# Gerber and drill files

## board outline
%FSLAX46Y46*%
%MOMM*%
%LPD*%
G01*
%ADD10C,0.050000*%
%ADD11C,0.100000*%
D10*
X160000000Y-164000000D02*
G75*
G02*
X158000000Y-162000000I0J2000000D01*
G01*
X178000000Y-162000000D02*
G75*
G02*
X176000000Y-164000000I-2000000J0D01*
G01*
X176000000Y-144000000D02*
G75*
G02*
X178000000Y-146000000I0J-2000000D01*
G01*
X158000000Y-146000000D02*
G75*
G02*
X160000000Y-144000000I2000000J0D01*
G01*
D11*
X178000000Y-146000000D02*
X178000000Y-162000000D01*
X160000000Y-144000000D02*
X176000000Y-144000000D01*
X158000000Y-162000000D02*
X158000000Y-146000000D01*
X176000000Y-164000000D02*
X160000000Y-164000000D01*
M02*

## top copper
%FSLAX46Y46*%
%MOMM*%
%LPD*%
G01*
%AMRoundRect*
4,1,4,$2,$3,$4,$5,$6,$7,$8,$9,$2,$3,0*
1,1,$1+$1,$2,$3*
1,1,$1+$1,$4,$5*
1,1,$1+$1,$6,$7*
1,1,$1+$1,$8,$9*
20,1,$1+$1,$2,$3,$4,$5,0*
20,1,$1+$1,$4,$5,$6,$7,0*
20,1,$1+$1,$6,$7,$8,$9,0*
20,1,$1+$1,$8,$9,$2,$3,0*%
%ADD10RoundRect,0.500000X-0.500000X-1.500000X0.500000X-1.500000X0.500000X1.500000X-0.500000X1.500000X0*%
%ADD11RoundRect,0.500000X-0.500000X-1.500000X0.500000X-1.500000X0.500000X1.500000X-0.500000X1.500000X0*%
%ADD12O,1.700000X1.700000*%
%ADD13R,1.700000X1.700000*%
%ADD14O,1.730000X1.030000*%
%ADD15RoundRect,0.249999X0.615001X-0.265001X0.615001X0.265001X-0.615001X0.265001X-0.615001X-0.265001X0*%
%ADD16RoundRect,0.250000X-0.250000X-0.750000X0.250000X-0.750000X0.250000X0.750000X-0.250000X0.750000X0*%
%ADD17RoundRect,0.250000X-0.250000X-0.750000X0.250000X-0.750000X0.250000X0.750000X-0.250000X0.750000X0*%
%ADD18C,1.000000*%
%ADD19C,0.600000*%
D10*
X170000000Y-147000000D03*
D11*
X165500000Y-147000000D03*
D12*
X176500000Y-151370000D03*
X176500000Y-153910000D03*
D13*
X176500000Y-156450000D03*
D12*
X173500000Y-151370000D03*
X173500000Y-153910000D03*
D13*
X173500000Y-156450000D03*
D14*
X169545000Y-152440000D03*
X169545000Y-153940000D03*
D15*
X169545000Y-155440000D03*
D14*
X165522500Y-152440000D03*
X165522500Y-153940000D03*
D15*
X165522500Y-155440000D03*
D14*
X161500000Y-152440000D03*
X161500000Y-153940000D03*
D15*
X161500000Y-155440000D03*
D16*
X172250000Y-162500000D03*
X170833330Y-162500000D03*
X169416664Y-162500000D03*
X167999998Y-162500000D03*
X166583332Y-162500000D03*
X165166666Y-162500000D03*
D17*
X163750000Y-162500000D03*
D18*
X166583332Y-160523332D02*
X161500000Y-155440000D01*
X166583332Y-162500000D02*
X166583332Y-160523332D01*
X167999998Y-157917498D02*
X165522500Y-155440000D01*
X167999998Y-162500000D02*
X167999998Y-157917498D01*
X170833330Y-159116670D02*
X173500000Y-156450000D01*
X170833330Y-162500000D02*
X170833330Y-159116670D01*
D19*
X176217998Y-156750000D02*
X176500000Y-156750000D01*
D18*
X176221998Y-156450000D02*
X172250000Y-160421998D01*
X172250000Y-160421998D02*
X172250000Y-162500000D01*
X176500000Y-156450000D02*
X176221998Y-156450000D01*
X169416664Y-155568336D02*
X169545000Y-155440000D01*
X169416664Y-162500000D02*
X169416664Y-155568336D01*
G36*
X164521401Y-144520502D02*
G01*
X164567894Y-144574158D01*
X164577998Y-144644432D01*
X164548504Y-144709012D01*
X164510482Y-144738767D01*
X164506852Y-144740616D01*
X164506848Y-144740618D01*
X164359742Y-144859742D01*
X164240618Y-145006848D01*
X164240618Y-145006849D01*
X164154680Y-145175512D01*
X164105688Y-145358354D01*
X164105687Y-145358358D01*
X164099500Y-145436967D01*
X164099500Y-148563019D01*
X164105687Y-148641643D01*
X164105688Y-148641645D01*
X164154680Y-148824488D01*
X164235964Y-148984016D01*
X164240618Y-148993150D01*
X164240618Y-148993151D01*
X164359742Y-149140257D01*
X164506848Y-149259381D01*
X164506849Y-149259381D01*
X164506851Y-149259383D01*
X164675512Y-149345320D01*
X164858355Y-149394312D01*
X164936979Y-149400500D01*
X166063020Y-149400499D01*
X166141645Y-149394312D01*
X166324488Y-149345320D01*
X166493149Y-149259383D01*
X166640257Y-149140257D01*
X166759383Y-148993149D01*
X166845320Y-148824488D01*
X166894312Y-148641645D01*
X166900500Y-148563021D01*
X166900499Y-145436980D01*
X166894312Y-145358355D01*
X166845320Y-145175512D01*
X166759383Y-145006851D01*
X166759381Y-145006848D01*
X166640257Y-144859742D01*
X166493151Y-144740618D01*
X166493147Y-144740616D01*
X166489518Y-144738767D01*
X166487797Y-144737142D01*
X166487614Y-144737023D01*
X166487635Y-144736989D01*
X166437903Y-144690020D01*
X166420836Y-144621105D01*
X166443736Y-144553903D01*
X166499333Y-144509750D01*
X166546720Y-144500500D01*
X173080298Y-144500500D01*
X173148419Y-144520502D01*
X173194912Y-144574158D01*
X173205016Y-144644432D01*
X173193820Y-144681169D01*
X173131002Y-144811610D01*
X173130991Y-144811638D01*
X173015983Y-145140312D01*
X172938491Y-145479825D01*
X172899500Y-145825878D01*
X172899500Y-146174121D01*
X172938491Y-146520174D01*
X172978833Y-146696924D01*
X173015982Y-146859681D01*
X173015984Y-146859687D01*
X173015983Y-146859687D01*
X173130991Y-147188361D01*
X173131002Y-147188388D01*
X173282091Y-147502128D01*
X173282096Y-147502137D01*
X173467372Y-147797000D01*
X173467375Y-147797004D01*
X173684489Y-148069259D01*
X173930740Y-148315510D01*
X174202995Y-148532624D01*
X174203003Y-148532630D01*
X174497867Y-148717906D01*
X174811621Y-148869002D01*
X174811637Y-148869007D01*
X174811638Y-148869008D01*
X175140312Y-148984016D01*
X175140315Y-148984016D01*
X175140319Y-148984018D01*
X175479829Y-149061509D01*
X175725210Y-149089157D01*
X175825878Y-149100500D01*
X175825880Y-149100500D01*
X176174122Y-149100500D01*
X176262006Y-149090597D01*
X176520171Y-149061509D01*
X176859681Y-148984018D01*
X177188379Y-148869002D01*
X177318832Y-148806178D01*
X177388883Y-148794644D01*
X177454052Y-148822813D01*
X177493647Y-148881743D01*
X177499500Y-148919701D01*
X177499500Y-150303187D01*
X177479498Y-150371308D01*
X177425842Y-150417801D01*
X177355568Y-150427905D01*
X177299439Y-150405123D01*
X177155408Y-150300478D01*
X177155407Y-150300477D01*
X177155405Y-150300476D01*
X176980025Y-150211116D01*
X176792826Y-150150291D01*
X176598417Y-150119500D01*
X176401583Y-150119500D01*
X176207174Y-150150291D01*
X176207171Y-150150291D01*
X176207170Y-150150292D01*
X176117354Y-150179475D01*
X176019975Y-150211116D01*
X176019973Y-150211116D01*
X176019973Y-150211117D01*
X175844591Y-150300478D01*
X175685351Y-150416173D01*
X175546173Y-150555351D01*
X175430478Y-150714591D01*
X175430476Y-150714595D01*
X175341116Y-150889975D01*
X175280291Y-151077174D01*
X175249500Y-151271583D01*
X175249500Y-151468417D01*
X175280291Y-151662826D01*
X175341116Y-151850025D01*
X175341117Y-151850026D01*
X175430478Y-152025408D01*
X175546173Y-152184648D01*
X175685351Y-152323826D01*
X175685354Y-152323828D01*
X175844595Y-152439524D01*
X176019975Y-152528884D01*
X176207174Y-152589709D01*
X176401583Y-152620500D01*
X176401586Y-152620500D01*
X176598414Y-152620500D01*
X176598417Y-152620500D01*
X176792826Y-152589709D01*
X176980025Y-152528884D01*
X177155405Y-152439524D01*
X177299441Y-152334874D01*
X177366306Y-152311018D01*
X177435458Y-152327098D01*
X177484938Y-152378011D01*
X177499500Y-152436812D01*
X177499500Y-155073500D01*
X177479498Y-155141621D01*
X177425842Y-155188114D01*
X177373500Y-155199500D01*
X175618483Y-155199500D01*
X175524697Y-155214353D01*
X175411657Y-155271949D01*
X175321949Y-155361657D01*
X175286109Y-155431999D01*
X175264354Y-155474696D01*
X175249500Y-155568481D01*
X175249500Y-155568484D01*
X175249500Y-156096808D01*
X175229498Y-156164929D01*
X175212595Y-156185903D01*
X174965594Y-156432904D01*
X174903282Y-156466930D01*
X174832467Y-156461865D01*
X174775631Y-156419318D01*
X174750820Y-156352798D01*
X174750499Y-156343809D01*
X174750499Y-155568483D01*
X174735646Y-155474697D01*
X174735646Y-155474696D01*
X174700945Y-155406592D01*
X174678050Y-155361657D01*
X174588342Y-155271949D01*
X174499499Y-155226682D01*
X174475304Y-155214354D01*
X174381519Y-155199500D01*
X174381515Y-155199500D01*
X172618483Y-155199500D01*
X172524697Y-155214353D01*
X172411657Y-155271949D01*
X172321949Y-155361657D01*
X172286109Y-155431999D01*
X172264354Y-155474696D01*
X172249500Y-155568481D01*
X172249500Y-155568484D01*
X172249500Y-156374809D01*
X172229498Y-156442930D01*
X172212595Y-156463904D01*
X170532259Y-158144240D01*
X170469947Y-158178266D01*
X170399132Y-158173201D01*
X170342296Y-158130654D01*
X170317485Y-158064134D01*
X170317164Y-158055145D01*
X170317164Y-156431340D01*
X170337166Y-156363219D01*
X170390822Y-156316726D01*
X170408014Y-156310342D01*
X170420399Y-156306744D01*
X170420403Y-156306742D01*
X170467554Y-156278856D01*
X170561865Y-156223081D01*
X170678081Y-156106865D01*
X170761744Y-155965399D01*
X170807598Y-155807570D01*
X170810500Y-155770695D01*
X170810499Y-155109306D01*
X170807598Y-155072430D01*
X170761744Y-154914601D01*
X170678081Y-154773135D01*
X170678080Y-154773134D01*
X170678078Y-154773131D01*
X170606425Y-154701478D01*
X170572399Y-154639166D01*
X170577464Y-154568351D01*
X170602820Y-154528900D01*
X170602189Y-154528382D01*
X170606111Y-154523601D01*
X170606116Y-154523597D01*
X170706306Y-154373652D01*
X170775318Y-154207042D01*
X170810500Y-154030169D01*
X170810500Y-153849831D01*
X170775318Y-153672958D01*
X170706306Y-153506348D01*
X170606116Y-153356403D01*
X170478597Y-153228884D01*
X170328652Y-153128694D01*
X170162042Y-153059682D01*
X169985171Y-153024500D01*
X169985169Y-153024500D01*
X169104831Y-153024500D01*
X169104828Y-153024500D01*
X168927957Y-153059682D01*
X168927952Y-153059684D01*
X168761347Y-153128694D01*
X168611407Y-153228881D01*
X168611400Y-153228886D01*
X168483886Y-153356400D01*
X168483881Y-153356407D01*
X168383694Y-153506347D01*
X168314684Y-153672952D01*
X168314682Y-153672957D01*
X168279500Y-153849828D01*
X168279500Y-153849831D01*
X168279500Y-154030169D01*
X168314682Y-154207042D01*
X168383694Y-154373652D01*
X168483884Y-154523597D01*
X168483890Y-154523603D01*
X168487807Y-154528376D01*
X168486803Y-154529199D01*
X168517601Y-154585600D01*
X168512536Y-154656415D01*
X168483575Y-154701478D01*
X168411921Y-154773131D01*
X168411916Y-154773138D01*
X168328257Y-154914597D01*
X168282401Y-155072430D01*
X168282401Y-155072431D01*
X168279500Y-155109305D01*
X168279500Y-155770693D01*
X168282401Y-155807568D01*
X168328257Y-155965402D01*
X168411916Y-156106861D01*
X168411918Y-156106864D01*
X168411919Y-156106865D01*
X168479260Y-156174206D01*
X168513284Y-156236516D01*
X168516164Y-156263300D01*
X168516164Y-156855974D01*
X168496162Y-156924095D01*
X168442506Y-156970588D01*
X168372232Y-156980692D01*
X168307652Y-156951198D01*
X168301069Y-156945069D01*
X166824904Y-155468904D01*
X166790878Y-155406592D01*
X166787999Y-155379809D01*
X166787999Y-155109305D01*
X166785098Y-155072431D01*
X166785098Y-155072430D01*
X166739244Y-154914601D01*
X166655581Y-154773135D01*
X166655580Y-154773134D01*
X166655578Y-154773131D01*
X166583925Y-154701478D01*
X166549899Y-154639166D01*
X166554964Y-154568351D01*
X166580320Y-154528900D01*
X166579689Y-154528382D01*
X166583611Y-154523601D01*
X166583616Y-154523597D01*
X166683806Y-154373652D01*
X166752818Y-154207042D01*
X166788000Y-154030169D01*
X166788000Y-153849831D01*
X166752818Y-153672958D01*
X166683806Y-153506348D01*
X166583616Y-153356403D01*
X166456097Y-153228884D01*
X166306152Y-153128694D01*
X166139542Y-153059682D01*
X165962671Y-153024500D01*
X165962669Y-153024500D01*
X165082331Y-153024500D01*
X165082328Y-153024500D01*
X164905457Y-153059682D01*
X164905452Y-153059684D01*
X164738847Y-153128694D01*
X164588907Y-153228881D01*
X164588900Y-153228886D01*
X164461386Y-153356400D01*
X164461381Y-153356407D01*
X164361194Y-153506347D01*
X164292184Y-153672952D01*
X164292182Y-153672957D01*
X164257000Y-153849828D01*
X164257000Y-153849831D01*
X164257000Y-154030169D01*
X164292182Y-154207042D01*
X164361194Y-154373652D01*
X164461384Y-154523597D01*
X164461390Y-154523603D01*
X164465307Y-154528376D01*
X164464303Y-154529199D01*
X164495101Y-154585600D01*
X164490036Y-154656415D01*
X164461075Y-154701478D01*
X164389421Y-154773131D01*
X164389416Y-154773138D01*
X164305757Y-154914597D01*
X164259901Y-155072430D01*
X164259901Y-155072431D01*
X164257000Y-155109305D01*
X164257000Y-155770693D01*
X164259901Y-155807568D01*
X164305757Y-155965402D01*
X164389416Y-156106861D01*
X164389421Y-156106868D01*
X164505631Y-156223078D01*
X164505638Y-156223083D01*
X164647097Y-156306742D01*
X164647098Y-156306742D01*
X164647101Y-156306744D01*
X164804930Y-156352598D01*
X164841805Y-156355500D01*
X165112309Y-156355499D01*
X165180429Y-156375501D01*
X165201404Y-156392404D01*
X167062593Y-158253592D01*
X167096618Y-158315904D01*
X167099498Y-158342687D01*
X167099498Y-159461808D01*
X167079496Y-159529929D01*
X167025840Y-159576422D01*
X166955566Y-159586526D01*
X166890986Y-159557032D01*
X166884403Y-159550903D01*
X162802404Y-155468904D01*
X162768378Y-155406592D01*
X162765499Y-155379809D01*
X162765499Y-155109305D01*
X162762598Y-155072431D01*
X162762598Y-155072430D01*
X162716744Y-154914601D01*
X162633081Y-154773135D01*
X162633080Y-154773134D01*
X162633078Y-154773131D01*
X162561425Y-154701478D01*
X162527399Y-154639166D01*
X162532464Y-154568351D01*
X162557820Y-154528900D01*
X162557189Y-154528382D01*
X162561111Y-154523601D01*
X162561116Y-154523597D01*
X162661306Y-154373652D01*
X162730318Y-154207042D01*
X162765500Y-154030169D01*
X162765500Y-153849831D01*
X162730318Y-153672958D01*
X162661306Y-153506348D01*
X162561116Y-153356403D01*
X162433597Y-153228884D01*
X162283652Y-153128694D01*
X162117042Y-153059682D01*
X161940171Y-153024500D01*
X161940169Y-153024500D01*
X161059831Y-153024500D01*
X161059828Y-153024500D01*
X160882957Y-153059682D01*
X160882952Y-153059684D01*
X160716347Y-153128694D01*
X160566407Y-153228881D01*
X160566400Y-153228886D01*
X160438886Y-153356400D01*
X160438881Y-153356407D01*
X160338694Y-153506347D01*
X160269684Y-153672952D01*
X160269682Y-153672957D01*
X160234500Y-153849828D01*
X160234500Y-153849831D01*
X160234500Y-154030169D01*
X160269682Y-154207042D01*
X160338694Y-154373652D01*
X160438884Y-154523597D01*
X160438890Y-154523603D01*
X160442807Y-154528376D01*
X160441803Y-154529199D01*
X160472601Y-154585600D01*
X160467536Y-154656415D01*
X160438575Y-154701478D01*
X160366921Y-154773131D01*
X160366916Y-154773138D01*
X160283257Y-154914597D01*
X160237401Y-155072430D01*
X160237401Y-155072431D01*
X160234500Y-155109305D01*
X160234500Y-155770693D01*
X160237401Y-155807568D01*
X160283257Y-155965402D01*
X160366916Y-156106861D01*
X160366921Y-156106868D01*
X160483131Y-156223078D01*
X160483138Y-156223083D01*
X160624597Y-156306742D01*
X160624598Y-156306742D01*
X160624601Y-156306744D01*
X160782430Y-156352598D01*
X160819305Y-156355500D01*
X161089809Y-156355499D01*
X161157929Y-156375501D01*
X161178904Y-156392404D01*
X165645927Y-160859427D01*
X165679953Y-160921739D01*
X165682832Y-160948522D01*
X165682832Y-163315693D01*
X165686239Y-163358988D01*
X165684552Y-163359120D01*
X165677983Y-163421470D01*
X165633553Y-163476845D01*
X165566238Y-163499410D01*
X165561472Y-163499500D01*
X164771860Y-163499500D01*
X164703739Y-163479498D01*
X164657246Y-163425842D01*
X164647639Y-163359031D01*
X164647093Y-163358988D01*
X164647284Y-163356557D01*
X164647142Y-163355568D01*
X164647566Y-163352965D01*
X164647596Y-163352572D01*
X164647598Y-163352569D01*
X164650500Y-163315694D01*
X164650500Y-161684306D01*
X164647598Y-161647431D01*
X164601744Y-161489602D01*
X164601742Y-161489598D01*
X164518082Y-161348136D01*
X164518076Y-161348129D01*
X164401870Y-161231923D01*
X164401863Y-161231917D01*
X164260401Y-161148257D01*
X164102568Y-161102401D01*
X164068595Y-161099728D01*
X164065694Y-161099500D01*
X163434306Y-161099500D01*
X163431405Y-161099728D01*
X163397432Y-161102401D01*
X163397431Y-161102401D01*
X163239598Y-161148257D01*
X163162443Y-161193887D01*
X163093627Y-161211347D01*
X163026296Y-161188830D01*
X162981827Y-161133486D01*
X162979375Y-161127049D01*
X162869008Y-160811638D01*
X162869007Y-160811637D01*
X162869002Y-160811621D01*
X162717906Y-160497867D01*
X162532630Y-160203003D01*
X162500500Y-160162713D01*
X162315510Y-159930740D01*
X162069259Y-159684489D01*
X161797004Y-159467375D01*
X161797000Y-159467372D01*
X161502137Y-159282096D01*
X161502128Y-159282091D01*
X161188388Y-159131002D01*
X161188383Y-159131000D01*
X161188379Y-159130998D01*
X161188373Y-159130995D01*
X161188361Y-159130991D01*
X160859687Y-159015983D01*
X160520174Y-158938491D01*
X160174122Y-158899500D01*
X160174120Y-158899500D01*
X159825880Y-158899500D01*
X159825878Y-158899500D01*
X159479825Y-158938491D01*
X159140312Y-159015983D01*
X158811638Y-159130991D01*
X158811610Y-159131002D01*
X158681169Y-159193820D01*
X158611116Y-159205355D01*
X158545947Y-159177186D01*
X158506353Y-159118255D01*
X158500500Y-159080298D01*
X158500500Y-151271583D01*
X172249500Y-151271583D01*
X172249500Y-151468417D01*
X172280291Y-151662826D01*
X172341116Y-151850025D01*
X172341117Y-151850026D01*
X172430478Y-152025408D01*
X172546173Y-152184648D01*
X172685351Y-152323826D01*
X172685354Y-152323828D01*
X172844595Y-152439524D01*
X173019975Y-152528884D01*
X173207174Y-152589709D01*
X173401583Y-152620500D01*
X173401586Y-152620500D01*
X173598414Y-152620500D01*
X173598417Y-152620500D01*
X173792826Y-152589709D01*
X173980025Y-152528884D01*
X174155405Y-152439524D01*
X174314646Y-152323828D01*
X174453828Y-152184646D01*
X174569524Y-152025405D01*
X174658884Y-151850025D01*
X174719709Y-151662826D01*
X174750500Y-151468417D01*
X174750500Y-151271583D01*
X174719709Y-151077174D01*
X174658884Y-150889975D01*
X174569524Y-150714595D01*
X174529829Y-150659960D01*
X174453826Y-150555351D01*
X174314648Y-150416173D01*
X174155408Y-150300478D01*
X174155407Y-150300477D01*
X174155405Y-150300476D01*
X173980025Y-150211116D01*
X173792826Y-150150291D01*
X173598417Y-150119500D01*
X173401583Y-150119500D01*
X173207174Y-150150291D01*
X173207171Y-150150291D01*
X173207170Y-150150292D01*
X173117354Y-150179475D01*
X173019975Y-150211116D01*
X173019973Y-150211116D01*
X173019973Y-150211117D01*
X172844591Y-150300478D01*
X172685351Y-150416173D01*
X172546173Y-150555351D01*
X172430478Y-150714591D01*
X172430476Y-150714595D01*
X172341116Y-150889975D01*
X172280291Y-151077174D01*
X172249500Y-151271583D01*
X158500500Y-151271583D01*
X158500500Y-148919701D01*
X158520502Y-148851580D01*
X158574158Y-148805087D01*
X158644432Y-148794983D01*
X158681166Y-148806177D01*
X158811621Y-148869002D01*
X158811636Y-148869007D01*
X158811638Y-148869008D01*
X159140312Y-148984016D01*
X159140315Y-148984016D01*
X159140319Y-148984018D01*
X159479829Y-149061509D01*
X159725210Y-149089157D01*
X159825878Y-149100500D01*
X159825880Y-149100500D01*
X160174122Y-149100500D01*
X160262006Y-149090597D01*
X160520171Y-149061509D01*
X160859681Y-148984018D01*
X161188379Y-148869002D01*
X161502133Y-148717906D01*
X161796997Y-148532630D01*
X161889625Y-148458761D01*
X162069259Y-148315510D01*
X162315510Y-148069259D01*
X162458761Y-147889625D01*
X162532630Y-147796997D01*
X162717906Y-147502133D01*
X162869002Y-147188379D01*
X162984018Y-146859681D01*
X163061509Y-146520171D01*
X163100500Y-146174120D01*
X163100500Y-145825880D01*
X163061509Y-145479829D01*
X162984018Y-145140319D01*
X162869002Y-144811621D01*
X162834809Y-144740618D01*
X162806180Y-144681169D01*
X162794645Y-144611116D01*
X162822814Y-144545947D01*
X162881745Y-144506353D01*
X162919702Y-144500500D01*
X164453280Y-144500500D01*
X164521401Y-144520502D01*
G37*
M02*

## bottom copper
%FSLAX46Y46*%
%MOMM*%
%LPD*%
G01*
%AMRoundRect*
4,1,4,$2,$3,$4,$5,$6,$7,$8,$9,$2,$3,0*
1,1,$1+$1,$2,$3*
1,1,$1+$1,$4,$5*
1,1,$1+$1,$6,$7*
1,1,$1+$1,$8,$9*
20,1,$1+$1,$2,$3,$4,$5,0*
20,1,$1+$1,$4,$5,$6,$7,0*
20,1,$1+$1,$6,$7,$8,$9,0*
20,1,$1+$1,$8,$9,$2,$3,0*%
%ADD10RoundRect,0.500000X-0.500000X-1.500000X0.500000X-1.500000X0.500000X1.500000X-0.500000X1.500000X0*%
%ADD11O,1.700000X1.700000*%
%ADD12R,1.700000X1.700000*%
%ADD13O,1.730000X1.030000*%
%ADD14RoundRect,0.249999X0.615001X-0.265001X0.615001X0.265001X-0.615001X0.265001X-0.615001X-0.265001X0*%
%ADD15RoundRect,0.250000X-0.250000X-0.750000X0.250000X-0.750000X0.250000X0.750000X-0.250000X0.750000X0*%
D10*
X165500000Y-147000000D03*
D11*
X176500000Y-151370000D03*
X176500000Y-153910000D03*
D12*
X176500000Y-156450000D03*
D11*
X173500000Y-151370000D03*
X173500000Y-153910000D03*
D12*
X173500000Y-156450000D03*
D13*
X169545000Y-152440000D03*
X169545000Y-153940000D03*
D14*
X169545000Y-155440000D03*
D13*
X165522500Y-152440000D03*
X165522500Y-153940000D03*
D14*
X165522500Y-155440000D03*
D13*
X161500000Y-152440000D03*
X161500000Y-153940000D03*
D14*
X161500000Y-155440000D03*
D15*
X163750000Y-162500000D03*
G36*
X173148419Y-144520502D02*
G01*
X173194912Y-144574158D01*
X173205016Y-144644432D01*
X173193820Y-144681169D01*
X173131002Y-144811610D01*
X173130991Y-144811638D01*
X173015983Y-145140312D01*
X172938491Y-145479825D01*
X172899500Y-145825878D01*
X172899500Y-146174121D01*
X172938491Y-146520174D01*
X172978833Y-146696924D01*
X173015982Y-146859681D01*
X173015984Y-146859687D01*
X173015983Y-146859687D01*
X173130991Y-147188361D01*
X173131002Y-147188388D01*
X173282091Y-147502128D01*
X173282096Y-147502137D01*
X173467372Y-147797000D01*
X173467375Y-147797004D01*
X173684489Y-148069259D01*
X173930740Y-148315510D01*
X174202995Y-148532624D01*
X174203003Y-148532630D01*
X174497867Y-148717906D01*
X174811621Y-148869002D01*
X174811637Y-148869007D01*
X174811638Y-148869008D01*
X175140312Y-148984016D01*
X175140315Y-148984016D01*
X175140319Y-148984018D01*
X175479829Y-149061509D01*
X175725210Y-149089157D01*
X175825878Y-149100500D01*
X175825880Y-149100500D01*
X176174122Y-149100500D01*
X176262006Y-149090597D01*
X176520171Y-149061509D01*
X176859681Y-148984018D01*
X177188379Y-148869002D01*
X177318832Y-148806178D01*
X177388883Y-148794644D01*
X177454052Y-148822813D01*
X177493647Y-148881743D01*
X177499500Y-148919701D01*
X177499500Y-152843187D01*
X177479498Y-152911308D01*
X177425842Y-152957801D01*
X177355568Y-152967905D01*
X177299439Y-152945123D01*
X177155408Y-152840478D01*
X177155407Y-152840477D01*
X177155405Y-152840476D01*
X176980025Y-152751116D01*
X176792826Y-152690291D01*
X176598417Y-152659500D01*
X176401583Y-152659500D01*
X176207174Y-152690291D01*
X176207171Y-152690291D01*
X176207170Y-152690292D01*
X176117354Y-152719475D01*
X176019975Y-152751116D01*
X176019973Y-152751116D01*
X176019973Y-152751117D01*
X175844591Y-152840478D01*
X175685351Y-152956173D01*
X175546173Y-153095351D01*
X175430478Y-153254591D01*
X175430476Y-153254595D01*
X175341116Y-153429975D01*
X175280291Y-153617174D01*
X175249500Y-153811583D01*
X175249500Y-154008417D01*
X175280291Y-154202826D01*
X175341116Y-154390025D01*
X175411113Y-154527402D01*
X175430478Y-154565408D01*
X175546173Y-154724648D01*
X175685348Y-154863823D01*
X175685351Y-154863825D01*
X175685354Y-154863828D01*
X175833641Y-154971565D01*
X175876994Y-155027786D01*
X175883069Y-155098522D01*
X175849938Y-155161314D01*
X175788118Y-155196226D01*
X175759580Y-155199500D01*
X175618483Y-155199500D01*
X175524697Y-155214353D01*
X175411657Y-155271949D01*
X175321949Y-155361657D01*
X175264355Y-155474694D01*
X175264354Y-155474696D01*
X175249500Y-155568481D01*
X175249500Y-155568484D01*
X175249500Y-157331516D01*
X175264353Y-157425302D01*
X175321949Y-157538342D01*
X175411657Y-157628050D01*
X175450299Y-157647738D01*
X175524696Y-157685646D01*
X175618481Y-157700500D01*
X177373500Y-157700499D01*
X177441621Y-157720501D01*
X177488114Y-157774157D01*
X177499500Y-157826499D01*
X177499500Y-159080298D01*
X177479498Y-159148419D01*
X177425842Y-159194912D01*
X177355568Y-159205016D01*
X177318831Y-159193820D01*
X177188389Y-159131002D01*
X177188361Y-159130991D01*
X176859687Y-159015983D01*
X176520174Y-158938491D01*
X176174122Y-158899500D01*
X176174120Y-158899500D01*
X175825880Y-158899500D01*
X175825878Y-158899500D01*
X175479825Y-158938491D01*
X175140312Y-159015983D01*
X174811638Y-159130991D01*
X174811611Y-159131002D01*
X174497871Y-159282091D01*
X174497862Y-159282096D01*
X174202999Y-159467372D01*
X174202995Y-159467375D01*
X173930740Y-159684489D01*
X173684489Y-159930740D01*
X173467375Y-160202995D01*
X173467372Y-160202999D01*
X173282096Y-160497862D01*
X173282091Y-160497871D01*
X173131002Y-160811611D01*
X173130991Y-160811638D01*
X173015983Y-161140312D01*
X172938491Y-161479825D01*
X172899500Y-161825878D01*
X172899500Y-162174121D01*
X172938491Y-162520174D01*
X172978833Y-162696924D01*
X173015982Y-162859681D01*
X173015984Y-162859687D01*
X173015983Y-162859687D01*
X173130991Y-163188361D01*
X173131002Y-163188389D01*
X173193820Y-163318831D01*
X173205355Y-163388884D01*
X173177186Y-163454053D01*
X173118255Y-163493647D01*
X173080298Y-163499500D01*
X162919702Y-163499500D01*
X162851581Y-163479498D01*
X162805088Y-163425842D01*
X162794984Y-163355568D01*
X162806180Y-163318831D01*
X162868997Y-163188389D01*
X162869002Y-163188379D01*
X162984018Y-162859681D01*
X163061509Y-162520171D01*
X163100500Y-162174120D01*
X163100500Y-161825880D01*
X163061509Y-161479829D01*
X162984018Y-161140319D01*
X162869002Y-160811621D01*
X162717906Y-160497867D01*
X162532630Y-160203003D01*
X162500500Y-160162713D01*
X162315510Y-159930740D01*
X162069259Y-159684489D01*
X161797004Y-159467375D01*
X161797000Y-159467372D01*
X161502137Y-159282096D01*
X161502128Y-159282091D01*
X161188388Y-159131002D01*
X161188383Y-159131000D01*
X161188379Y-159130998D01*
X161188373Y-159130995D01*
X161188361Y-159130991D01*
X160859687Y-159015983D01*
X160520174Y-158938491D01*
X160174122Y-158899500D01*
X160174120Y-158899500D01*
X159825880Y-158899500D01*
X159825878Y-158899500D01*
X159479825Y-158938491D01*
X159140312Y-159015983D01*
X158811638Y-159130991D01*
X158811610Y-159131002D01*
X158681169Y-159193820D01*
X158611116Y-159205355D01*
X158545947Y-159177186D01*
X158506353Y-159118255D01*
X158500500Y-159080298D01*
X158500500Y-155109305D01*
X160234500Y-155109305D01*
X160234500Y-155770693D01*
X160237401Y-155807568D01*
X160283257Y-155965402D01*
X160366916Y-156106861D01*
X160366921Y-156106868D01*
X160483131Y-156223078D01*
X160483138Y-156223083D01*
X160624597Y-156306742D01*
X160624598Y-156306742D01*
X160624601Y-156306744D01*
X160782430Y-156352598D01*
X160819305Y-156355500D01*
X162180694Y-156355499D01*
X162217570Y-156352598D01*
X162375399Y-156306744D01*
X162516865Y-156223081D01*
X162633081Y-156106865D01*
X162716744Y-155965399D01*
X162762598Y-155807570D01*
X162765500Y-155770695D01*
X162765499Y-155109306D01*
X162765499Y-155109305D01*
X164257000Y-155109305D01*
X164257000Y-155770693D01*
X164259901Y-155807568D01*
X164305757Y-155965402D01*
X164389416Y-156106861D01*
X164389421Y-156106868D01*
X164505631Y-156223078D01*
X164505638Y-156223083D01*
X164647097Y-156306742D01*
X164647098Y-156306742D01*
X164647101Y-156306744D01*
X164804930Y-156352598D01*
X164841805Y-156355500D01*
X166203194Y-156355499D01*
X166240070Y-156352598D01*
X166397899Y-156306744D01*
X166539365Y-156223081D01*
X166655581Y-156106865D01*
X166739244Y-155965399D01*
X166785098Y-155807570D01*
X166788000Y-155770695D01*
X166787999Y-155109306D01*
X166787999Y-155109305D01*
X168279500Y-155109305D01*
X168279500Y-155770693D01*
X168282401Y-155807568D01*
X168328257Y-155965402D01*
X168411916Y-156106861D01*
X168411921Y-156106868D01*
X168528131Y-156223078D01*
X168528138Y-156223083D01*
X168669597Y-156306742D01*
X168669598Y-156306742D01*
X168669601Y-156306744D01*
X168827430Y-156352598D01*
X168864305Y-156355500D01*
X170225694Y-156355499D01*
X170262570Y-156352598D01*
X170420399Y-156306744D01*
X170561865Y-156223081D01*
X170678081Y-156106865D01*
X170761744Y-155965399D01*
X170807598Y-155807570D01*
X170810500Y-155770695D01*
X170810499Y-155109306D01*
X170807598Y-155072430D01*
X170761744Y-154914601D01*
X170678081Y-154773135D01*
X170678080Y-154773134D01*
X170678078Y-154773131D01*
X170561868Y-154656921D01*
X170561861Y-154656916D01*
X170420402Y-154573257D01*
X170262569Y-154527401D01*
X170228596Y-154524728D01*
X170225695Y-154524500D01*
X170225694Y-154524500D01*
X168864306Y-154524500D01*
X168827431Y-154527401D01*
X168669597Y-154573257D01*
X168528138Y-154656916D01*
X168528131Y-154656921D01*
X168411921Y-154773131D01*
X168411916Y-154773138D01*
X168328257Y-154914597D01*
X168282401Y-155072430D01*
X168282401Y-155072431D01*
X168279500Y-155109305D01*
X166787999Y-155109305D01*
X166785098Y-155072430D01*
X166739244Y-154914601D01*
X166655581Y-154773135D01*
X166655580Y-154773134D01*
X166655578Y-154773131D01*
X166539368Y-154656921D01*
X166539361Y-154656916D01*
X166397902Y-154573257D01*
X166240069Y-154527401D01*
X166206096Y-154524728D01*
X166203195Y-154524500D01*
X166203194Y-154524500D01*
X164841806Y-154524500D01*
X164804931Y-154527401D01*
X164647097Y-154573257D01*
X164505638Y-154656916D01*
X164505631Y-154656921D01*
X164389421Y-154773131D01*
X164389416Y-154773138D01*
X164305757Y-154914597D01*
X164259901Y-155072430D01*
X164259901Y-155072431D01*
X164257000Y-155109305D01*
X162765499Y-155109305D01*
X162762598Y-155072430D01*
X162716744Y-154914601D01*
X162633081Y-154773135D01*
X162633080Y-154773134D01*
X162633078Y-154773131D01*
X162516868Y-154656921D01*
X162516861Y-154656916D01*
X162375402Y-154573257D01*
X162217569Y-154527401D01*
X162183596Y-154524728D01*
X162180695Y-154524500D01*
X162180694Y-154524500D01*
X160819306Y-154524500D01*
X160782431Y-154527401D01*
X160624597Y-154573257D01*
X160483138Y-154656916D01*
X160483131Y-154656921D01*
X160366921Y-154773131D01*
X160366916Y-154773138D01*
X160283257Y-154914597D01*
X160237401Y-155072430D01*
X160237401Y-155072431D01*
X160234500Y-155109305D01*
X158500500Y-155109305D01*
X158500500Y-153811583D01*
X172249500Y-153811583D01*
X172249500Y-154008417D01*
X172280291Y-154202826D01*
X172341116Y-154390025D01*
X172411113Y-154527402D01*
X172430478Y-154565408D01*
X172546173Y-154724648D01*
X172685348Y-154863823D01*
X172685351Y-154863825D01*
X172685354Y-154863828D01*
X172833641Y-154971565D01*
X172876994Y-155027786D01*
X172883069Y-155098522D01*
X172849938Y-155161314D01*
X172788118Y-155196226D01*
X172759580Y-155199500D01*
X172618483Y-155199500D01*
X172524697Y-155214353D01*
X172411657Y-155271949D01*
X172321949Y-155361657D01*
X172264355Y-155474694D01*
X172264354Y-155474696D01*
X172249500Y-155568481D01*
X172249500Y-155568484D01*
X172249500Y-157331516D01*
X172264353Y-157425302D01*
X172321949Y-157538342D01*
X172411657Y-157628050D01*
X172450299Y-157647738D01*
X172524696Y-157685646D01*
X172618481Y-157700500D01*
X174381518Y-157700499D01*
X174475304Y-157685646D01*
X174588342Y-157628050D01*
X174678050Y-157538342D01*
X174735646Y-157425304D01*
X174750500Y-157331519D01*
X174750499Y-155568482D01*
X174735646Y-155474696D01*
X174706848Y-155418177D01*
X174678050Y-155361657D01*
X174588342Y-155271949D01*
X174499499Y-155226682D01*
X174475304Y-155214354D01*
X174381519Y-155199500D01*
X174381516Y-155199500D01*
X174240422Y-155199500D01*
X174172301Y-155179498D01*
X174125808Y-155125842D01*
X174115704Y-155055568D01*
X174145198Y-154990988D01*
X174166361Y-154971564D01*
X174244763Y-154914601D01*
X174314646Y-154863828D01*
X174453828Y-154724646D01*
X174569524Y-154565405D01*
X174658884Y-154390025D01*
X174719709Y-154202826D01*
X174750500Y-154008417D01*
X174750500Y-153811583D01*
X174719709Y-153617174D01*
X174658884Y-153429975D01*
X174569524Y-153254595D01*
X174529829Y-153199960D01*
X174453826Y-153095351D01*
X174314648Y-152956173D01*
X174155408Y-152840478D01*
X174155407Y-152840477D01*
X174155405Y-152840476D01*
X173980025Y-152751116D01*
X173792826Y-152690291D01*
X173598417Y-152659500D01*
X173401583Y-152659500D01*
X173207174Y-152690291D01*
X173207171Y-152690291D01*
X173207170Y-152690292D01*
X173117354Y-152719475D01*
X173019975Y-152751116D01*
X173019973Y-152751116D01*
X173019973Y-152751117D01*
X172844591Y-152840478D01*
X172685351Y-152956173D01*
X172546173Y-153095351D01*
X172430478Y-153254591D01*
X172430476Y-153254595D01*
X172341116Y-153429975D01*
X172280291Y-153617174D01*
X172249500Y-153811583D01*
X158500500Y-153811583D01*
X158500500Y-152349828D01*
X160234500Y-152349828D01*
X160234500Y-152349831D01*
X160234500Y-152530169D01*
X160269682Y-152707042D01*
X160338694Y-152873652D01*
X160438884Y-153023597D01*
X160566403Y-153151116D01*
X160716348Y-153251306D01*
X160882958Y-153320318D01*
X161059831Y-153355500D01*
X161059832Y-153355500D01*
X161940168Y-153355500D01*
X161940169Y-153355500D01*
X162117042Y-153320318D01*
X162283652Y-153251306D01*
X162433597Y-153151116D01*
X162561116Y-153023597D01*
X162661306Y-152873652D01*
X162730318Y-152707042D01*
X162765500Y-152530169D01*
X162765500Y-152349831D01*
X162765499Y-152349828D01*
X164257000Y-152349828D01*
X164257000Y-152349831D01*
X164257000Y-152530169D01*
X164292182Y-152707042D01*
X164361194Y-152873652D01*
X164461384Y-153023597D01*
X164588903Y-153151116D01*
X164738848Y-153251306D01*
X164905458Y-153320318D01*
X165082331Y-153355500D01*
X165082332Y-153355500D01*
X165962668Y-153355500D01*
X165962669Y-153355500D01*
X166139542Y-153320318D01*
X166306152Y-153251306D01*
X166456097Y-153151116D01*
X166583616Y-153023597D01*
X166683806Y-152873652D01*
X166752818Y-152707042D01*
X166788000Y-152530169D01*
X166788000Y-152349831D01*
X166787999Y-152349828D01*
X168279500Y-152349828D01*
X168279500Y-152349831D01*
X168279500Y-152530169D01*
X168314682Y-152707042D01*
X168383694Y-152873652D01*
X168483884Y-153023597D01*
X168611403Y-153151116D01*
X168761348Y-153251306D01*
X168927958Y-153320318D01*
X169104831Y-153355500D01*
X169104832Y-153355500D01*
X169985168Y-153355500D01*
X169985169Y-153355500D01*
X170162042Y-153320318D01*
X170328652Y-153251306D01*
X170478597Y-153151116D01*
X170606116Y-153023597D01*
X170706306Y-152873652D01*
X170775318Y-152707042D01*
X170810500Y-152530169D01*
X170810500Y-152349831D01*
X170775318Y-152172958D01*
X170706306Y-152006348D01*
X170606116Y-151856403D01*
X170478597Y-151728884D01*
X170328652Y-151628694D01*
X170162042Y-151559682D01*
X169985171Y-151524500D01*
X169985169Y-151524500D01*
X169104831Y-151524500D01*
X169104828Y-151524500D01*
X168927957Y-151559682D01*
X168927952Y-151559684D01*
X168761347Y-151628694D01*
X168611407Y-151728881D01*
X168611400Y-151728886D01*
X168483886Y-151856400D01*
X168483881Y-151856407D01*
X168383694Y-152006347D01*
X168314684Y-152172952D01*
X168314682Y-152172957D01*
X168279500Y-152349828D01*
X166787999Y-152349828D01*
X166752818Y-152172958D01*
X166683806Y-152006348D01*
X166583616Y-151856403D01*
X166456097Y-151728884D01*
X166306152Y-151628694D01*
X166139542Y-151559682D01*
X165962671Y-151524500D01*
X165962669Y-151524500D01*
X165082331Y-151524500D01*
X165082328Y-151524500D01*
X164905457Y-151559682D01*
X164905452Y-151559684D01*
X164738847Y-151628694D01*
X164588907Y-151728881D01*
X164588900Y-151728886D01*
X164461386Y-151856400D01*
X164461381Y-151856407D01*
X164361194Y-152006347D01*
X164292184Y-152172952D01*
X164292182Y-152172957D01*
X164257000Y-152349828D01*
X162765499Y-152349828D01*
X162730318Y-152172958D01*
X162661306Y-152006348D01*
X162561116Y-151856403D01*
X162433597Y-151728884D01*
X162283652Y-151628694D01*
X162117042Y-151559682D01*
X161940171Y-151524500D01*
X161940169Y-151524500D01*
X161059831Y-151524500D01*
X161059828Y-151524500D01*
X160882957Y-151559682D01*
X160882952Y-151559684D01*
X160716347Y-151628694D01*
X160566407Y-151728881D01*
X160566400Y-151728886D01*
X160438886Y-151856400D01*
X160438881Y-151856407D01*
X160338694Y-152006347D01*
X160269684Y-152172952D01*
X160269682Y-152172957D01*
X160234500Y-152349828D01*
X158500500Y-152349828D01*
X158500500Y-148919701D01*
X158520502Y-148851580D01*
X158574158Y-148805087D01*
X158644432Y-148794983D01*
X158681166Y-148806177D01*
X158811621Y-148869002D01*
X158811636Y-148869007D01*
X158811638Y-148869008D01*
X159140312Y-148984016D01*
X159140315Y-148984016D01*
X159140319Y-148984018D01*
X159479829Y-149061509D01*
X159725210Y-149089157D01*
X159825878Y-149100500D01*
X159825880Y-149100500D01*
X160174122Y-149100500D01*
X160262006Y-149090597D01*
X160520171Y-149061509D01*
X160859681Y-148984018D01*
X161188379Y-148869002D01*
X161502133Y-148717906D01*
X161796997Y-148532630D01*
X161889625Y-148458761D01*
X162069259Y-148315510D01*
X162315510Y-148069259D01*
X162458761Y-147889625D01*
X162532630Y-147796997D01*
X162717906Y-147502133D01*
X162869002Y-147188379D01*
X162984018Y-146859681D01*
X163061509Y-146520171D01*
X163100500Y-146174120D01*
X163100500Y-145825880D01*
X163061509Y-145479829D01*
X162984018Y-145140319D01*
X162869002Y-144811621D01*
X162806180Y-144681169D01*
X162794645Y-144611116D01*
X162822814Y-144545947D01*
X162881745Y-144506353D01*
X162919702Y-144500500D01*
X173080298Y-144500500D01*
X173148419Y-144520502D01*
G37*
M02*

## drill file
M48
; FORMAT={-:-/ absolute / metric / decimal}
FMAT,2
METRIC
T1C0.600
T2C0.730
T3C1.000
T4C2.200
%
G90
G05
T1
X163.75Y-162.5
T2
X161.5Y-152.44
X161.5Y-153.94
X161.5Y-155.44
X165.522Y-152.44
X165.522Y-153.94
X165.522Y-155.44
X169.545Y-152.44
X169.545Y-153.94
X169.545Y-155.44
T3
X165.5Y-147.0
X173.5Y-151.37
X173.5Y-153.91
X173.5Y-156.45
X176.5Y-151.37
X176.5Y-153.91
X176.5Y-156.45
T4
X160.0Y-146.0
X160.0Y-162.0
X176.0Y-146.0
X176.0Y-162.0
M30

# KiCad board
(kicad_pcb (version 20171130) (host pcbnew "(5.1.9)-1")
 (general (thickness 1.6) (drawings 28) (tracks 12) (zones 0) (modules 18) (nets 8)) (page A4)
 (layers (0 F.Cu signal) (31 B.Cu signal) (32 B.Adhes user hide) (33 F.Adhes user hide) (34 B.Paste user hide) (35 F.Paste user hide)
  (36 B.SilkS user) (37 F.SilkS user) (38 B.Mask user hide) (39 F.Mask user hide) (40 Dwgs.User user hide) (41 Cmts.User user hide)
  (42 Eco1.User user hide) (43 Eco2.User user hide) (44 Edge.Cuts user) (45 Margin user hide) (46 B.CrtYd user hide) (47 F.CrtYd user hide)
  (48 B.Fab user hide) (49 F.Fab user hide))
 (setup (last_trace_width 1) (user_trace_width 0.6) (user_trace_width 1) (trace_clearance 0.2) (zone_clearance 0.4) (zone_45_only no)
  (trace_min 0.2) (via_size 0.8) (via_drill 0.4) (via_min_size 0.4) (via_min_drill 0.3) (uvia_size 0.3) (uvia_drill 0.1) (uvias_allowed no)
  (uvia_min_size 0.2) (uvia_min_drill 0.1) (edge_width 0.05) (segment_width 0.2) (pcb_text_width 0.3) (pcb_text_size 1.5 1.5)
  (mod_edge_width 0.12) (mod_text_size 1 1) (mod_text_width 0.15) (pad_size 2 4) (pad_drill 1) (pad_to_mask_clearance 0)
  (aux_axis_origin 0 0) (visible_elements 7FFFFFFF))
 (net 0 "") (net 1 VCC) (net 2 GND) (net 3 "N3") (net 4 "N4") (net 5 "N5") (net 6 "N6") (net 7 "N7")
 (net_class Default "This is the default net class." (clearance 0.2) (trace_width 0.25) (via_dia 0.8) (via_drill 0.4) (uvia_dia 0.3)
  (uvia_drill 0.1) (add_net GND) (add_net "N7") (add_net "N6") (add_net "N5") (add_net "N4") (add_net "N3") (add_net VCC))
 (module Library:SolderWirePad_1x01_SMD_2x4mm (layer F.Cu) (at 170 147)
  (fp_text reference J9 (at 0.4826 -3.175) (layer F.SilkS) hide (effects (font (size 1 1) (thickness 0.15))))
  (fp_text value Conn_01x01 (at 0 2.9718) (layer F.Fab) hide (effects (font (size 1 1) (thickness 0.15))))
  (pad 1 smd roundrect (at 0 0) (size 2 4) (layers F.Cu F.Paste F.Mask) (roundrect_rratio 0.25) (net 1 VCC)))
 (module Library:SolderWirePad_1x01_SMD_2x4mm (layer F.Cu) (at 165.5 147)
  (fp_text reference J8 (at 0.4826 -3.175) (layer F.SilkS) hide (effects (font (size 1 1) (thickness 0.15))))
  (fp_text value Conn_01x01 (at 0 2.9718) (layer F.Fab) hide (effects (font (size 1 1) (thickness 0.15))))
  (pad 1 thru_hole roundrect (at 0 0) (size 2 4) (drill 1) (layers *.Cu *.Mask) (roundrect_rratio 0.25) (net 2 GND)))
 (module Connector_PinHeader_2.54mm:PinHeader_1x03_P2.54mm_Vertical (layer F.Cu) (at 176.5 156.45 180)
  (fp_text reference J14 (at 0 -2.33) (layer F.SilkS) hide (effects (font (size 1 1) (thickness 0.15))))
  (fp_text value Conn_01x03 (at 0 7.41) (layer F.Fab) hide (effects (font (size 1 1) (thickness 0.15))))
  (pad 3 thru_hole oval (at 0 5.08 180) (size 1.7 1.7) (drill 1) (layers *.Cu *.Mask) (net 2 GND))
  (pad 2 thru_hole oval (at 0 2.54 180) (size 1.7 1.7) (drill 1) (layers *.Cu *.Mask) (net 1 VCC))
  (pad 1 thru_hole rect (at 0 0 180) (size 1.7 1.7) (drill 1) (layers *.Cu *.Mask) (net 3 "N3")))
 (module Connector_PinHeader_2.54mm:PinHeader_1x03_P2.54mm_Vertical (layer F.Cu) (at 173.5 156.45 180)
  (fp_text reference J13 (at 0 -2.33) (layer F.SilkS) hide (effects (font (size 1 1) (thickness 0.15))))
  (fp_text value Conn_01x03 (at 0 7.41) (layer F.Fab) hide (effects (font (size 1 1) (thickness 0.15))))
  (pad 3 thru_hole oval (at 0 5.08 180) (size 1.7 1.7) (drill 1) (layers *.Cu *.Mask) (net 2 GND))
  (pad 2 thru_hole oval (at 0 2.54 180) (size 1.7 1.7) (drill 1) (layers *.Cu *.Mask) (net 1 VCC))
  (pad 1 thru_hole rect (at 0 0 180) (size 1.7 1.7) (drill 1) (layers *.Cu *.Mask) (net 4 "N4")))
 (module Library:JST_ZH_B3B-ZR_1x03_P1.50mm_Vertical (layer F.Cu) (at 169.545 155.44 90)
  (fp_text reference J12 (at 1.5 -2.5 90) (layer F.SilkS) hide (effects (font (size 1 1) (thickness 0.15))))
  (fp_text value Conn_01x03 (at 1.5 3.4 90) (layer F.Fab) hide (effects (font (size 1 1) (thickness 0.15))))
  (pad 3 thru_hole oval (at 3 0 90) (size 1.03 1.73) (drill 0.73) (layers *.Cu *.Mask) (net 1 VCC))
  (pad 2 thru_hole oval (at 1.5 0 90) (size 1.03 1.73) (drill 0.73) (layers *.Cu *.Mask) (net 2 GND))
  (pad 1 thru_hole roundrect (at 0 0 90) (size 1.03 1.73) (drill 0.73) (layers *.Cu *.Mask) (roundrect_rratio 0.2427174757281553)
   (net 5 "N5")))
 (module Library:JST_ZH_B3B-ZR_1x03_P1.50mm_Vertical (layer F.Cu) (at 165.5225 155.44 90)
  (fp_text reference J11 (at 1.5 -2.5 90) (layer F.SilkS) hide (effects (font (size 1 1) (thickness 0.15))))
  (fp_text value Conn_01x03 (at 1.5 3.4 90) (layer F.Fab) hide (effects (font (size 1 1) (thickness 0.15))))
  (pad 3 thru_hole oval (at 3 0 90) (size 1.03 1.73) (drill 0.73) (layers *.Cu *.Mask) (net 1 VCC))
  (pad 2 thru_hole oval (at 1.5 0 90) (size 1.03 1.73) (drill 0.73) (layers *.Cu *.Mask) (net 2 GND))
  (pad 1 thru_hole roundrect (at 0 0 90) (size 1.03 1.73) (drill 0.73) (layers *.Cu *.Mask) (roundrect_rratio 0.2427174757281553)
   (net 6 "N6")))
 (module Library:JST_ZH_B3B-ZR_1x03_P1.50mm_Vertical (layer F.Cu) (at 161.5 155.44 90)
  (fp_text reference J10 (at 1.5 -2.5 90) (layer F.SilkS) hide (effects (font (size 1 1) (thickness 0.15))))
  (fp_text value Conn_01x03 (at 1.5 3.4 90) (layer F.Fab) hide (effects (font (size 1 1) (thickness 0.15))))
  (pad 3 thru_hole oval (at 3 0 90) (size 1.03 1.73) (drill 0.73) (layers *.Cu *.Mask) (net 1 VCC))
  (pad 2 thru_hole oval (at 1.5 0 90) (size 1.03 1.73) (drill 0.73) (layers *.Cu *.Mask) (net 2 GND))
  (pad 1 thru_hole roundrect (at 0 0 90) (size 1.03 1.73) (drill 0.73) (layers *.Cu *.Mask) (roundrect_rratio 0.2427174757281553)
   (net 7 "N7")))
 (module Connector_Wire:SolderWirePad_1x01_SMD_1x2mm (layer F.Cu) (at 172.25 162.5)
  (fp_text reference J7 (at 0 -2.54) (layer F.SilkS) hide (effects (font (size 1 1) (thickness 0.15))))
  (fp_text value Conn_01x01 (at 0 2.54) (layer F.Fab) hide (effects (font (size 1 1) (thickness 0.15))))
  (pad 1 smd roundrect (at 0 0) (size 1 2) (layers F.Cu F.Paste F.Mask) (roundrect_rratio 0.25) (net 3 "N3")))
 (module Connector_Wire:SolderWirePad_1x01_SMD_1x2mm (layer F.Cu) (at 170.83333 162.5)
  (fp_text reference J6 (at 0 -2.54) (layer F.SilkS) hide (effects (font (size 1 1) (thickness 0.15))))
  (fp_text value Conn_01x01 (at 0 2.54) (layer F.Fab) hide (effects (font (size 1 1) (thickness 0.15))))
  (pad 1 smd roundrect (at 0 0) (size 1 2) (layers F.Cu F.Paste F.Mask) (roundrect_rratio 0.25) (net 4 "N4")))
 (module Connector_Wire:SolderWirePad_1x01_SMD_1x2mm (layer F.Cu) (at 169.416664 162.5)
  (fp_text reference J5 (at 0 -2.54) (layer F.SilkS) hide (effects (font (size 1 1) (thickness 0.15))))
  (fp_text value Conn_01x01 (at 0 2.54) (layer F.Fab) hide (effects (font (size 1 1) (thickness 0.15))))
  (pad 1 smd roundrect (at 0 0) (size 1 2) (layers F.Cu F.Paste F.Mask) (roundrect_rratio 0.25) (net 5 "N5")))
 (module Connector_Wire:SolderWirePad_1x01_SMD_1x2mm (layer F.Cu) (at 167.999998 162.5)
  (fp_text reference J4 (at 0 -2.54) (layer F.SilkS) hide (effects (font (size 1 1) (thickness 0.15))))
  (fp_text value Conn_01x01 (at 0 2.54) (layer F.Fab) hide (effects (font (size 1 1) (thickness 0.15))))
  (pad 1 smd roundrect (at 0 0) (size 1 2) (layers F.Cu F.Paste F.Mask) (roundrect_rratio 0.25) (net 6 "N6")))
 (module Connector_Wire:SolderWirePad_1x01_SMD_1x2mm (layer F.Cu) (at 166.583332 162.5)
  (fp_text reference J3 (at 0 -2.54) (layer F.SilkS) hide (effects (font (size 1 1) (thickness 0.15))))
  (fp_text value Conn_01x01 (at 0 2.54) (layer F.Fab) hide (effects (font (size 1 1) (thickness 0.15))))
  (pad 1 smd roundrect (at 0 0) (size 1 2) (layers F.Cu F.Paste F.Mask) (roundrect_rratio 0.25) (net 7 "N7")))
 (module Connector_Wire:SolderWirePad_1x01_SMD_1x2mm (layer F.Cu) (at 165.166666 162.5)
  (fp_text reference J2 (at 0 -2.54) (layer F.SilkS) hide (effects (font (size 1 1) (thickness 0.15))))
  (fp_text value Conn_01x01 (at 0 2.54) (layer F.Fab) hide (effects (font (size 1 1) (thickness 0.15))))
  (pad 1 smd roundrect (at 0 0) (size 1 2) (layers F.Cu F.Paste F.Mask) (roundrect_rratio 0.25) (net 1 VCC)))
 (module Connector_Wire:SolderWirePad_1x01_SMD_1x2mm (layer F.Cu) (at 163.75 162.5)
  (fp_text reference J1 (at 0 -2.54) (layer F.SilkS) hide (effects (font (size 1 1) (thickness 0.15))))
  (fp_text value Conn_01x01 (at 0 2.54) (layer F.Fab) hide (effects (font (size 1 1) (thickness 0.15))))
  (pad 1 thru_hole roundrect (at 0 0) (size 1 2) (drill 0.6) (layers *.Cu *.Mask) (roundrect_rratio 0.25) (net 2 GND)))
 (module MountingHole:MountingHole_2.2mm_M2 (layer F.Cu) (at 176 162)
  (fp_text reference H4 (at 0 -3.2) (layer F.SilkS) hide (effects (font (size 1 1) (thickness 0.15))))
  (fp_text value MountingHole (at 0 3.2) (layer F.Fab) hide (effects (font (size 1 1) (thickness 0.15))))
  (pad "" np_thru_hole circle (at 0 0) (size 2.2 2.2) (drill 2.2) (layers *.Cu *.Mask) (clearance 2)))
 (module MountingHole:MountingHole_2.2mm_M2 (layer F.Cu) (at 176 146)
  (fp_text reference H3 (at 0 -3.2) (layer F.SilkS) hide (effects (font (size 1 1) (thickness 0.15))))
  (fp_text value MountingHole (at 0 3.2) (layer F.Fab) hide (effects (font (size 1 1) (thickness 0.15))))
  (pad "" np_thru_hole circle (at 0 0) (size 2.2 2.2) (drill 2.2) (layers *.Cu *.Mask) (clearance 2)))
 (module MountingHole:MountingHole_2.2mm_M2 (layer F.Cu) (at 160 162)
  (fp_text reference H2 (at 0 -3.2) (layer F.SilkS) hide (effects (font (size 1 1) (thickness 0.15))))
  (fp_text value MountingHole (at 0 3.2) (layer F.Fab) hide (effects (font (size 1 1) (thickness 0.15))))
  (pad "" np_thru_hole circle (at 0 0) (size 2.2 2.2) (drill 2.2) (layers *.Cu *.Mask) (clearance 2)))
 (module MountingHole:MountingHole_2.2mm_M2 (layer F.Cu) (at 160 146)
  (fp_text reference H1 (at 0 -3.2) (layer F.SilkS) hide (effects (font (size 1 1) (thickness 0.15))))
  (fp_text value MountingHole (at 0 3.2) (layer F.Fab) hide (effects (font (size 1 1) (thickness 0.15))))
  (pad "" np_thru_hole circle (at 0 0) (size 2.2 2.2) (drill 2.2) (layers *.Cu *.Mask) (clearance 2)))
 (gr_arc (start 160 162) (end 158 162) (angle -90) (layer Edge.Cuts) (width 0.05))
 (gr_arc (start 176 162) (end 176 164) (angle -90) (layer Edge.Cuts) (width 0.05))
 (gr_arc (start 176 146) (end 178 146) (angle -90) (layer Edge.Cuts) (width 0.05))
 (gr_arc (start 160 146) (end 160 144) (angle -90) (layer Edge.Cuts) (width 0.05))
 (gr_line (start 178 146) (end 178 162) (layer Edge.Cuts) (width 0.1))
 (gr_line (start 160 144) (end 176 144) (layer Edge.Cuts) (width 0.1))
 (gr_line (start 158 162) (end 158 146) (layer Edge.Cuts) (width 0.1))
 (gr_line (start 176 164) (end 160 164) (layer Edge.Cuts) (width 0.1))
 (segment (start 166.583332 160.523332) (end 161.5 155.44) (width 1) (layer F.Cu) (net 7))
 (segment (start 166.583332 162.5) (end 166.583332 160.523332) (width 1) (layer F.Cu) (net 7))
 (segment (start 167.999998 157.917498) (end 165.5225 155.44) (width 1) (layer F.Cu) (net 6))
 (segment (start 167.999998 162.5) (end 167.999998 157.917498) (width 1) (layer F.Cu) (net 6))
 (segment (start 170.83333 159.11667) (end 173.5 156.45) (width 1) (layer F.Cu) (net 4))
 (segment (start 170.83333 162.5) (end 170.83333 159.11667) (width 1) (layer F.Cu) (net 4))
 (segment (start 176.217998 156.75) (end 176.5 156.75) (width 0.6) (layer F.Cu) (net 3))
 (segment (start 176.221998 156.45) (end 172.25 160.421998) (width 1) (layer F.Cu) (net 3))
 (segment (start 172.25 160.421998) (end 172.25 162.5) (width 1) (layer F.Cu) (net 3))
 (segment (start 176.5 156.45) (end 176.221998 156.45) (width 1) (layer F.Cu) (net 3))
 (segment (start 169.416664 155.568336) (end 169.545 155.44) (width 1) (layer F.Cu) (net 5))
 (segment (start 169.416664 162.5) (end 169.416664 155.568336) (width 1) (layer F.Cu) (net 5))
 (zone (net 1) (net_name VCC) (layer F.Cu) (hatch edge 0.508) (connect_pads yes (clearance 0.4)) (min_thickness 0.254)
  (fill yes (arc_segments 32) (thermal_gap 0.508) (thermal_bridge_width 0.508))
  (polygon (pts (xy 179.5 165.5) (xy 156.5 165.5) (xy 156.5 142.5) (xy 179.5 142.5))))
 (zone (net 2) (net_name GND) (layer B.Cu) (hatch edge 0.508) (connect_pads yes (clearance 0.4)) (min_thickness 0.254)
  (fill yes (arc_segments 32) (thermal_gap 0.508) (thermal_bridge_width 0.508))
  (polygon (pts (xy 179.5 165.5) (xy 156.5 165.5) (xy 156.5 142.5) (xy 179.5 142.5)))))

